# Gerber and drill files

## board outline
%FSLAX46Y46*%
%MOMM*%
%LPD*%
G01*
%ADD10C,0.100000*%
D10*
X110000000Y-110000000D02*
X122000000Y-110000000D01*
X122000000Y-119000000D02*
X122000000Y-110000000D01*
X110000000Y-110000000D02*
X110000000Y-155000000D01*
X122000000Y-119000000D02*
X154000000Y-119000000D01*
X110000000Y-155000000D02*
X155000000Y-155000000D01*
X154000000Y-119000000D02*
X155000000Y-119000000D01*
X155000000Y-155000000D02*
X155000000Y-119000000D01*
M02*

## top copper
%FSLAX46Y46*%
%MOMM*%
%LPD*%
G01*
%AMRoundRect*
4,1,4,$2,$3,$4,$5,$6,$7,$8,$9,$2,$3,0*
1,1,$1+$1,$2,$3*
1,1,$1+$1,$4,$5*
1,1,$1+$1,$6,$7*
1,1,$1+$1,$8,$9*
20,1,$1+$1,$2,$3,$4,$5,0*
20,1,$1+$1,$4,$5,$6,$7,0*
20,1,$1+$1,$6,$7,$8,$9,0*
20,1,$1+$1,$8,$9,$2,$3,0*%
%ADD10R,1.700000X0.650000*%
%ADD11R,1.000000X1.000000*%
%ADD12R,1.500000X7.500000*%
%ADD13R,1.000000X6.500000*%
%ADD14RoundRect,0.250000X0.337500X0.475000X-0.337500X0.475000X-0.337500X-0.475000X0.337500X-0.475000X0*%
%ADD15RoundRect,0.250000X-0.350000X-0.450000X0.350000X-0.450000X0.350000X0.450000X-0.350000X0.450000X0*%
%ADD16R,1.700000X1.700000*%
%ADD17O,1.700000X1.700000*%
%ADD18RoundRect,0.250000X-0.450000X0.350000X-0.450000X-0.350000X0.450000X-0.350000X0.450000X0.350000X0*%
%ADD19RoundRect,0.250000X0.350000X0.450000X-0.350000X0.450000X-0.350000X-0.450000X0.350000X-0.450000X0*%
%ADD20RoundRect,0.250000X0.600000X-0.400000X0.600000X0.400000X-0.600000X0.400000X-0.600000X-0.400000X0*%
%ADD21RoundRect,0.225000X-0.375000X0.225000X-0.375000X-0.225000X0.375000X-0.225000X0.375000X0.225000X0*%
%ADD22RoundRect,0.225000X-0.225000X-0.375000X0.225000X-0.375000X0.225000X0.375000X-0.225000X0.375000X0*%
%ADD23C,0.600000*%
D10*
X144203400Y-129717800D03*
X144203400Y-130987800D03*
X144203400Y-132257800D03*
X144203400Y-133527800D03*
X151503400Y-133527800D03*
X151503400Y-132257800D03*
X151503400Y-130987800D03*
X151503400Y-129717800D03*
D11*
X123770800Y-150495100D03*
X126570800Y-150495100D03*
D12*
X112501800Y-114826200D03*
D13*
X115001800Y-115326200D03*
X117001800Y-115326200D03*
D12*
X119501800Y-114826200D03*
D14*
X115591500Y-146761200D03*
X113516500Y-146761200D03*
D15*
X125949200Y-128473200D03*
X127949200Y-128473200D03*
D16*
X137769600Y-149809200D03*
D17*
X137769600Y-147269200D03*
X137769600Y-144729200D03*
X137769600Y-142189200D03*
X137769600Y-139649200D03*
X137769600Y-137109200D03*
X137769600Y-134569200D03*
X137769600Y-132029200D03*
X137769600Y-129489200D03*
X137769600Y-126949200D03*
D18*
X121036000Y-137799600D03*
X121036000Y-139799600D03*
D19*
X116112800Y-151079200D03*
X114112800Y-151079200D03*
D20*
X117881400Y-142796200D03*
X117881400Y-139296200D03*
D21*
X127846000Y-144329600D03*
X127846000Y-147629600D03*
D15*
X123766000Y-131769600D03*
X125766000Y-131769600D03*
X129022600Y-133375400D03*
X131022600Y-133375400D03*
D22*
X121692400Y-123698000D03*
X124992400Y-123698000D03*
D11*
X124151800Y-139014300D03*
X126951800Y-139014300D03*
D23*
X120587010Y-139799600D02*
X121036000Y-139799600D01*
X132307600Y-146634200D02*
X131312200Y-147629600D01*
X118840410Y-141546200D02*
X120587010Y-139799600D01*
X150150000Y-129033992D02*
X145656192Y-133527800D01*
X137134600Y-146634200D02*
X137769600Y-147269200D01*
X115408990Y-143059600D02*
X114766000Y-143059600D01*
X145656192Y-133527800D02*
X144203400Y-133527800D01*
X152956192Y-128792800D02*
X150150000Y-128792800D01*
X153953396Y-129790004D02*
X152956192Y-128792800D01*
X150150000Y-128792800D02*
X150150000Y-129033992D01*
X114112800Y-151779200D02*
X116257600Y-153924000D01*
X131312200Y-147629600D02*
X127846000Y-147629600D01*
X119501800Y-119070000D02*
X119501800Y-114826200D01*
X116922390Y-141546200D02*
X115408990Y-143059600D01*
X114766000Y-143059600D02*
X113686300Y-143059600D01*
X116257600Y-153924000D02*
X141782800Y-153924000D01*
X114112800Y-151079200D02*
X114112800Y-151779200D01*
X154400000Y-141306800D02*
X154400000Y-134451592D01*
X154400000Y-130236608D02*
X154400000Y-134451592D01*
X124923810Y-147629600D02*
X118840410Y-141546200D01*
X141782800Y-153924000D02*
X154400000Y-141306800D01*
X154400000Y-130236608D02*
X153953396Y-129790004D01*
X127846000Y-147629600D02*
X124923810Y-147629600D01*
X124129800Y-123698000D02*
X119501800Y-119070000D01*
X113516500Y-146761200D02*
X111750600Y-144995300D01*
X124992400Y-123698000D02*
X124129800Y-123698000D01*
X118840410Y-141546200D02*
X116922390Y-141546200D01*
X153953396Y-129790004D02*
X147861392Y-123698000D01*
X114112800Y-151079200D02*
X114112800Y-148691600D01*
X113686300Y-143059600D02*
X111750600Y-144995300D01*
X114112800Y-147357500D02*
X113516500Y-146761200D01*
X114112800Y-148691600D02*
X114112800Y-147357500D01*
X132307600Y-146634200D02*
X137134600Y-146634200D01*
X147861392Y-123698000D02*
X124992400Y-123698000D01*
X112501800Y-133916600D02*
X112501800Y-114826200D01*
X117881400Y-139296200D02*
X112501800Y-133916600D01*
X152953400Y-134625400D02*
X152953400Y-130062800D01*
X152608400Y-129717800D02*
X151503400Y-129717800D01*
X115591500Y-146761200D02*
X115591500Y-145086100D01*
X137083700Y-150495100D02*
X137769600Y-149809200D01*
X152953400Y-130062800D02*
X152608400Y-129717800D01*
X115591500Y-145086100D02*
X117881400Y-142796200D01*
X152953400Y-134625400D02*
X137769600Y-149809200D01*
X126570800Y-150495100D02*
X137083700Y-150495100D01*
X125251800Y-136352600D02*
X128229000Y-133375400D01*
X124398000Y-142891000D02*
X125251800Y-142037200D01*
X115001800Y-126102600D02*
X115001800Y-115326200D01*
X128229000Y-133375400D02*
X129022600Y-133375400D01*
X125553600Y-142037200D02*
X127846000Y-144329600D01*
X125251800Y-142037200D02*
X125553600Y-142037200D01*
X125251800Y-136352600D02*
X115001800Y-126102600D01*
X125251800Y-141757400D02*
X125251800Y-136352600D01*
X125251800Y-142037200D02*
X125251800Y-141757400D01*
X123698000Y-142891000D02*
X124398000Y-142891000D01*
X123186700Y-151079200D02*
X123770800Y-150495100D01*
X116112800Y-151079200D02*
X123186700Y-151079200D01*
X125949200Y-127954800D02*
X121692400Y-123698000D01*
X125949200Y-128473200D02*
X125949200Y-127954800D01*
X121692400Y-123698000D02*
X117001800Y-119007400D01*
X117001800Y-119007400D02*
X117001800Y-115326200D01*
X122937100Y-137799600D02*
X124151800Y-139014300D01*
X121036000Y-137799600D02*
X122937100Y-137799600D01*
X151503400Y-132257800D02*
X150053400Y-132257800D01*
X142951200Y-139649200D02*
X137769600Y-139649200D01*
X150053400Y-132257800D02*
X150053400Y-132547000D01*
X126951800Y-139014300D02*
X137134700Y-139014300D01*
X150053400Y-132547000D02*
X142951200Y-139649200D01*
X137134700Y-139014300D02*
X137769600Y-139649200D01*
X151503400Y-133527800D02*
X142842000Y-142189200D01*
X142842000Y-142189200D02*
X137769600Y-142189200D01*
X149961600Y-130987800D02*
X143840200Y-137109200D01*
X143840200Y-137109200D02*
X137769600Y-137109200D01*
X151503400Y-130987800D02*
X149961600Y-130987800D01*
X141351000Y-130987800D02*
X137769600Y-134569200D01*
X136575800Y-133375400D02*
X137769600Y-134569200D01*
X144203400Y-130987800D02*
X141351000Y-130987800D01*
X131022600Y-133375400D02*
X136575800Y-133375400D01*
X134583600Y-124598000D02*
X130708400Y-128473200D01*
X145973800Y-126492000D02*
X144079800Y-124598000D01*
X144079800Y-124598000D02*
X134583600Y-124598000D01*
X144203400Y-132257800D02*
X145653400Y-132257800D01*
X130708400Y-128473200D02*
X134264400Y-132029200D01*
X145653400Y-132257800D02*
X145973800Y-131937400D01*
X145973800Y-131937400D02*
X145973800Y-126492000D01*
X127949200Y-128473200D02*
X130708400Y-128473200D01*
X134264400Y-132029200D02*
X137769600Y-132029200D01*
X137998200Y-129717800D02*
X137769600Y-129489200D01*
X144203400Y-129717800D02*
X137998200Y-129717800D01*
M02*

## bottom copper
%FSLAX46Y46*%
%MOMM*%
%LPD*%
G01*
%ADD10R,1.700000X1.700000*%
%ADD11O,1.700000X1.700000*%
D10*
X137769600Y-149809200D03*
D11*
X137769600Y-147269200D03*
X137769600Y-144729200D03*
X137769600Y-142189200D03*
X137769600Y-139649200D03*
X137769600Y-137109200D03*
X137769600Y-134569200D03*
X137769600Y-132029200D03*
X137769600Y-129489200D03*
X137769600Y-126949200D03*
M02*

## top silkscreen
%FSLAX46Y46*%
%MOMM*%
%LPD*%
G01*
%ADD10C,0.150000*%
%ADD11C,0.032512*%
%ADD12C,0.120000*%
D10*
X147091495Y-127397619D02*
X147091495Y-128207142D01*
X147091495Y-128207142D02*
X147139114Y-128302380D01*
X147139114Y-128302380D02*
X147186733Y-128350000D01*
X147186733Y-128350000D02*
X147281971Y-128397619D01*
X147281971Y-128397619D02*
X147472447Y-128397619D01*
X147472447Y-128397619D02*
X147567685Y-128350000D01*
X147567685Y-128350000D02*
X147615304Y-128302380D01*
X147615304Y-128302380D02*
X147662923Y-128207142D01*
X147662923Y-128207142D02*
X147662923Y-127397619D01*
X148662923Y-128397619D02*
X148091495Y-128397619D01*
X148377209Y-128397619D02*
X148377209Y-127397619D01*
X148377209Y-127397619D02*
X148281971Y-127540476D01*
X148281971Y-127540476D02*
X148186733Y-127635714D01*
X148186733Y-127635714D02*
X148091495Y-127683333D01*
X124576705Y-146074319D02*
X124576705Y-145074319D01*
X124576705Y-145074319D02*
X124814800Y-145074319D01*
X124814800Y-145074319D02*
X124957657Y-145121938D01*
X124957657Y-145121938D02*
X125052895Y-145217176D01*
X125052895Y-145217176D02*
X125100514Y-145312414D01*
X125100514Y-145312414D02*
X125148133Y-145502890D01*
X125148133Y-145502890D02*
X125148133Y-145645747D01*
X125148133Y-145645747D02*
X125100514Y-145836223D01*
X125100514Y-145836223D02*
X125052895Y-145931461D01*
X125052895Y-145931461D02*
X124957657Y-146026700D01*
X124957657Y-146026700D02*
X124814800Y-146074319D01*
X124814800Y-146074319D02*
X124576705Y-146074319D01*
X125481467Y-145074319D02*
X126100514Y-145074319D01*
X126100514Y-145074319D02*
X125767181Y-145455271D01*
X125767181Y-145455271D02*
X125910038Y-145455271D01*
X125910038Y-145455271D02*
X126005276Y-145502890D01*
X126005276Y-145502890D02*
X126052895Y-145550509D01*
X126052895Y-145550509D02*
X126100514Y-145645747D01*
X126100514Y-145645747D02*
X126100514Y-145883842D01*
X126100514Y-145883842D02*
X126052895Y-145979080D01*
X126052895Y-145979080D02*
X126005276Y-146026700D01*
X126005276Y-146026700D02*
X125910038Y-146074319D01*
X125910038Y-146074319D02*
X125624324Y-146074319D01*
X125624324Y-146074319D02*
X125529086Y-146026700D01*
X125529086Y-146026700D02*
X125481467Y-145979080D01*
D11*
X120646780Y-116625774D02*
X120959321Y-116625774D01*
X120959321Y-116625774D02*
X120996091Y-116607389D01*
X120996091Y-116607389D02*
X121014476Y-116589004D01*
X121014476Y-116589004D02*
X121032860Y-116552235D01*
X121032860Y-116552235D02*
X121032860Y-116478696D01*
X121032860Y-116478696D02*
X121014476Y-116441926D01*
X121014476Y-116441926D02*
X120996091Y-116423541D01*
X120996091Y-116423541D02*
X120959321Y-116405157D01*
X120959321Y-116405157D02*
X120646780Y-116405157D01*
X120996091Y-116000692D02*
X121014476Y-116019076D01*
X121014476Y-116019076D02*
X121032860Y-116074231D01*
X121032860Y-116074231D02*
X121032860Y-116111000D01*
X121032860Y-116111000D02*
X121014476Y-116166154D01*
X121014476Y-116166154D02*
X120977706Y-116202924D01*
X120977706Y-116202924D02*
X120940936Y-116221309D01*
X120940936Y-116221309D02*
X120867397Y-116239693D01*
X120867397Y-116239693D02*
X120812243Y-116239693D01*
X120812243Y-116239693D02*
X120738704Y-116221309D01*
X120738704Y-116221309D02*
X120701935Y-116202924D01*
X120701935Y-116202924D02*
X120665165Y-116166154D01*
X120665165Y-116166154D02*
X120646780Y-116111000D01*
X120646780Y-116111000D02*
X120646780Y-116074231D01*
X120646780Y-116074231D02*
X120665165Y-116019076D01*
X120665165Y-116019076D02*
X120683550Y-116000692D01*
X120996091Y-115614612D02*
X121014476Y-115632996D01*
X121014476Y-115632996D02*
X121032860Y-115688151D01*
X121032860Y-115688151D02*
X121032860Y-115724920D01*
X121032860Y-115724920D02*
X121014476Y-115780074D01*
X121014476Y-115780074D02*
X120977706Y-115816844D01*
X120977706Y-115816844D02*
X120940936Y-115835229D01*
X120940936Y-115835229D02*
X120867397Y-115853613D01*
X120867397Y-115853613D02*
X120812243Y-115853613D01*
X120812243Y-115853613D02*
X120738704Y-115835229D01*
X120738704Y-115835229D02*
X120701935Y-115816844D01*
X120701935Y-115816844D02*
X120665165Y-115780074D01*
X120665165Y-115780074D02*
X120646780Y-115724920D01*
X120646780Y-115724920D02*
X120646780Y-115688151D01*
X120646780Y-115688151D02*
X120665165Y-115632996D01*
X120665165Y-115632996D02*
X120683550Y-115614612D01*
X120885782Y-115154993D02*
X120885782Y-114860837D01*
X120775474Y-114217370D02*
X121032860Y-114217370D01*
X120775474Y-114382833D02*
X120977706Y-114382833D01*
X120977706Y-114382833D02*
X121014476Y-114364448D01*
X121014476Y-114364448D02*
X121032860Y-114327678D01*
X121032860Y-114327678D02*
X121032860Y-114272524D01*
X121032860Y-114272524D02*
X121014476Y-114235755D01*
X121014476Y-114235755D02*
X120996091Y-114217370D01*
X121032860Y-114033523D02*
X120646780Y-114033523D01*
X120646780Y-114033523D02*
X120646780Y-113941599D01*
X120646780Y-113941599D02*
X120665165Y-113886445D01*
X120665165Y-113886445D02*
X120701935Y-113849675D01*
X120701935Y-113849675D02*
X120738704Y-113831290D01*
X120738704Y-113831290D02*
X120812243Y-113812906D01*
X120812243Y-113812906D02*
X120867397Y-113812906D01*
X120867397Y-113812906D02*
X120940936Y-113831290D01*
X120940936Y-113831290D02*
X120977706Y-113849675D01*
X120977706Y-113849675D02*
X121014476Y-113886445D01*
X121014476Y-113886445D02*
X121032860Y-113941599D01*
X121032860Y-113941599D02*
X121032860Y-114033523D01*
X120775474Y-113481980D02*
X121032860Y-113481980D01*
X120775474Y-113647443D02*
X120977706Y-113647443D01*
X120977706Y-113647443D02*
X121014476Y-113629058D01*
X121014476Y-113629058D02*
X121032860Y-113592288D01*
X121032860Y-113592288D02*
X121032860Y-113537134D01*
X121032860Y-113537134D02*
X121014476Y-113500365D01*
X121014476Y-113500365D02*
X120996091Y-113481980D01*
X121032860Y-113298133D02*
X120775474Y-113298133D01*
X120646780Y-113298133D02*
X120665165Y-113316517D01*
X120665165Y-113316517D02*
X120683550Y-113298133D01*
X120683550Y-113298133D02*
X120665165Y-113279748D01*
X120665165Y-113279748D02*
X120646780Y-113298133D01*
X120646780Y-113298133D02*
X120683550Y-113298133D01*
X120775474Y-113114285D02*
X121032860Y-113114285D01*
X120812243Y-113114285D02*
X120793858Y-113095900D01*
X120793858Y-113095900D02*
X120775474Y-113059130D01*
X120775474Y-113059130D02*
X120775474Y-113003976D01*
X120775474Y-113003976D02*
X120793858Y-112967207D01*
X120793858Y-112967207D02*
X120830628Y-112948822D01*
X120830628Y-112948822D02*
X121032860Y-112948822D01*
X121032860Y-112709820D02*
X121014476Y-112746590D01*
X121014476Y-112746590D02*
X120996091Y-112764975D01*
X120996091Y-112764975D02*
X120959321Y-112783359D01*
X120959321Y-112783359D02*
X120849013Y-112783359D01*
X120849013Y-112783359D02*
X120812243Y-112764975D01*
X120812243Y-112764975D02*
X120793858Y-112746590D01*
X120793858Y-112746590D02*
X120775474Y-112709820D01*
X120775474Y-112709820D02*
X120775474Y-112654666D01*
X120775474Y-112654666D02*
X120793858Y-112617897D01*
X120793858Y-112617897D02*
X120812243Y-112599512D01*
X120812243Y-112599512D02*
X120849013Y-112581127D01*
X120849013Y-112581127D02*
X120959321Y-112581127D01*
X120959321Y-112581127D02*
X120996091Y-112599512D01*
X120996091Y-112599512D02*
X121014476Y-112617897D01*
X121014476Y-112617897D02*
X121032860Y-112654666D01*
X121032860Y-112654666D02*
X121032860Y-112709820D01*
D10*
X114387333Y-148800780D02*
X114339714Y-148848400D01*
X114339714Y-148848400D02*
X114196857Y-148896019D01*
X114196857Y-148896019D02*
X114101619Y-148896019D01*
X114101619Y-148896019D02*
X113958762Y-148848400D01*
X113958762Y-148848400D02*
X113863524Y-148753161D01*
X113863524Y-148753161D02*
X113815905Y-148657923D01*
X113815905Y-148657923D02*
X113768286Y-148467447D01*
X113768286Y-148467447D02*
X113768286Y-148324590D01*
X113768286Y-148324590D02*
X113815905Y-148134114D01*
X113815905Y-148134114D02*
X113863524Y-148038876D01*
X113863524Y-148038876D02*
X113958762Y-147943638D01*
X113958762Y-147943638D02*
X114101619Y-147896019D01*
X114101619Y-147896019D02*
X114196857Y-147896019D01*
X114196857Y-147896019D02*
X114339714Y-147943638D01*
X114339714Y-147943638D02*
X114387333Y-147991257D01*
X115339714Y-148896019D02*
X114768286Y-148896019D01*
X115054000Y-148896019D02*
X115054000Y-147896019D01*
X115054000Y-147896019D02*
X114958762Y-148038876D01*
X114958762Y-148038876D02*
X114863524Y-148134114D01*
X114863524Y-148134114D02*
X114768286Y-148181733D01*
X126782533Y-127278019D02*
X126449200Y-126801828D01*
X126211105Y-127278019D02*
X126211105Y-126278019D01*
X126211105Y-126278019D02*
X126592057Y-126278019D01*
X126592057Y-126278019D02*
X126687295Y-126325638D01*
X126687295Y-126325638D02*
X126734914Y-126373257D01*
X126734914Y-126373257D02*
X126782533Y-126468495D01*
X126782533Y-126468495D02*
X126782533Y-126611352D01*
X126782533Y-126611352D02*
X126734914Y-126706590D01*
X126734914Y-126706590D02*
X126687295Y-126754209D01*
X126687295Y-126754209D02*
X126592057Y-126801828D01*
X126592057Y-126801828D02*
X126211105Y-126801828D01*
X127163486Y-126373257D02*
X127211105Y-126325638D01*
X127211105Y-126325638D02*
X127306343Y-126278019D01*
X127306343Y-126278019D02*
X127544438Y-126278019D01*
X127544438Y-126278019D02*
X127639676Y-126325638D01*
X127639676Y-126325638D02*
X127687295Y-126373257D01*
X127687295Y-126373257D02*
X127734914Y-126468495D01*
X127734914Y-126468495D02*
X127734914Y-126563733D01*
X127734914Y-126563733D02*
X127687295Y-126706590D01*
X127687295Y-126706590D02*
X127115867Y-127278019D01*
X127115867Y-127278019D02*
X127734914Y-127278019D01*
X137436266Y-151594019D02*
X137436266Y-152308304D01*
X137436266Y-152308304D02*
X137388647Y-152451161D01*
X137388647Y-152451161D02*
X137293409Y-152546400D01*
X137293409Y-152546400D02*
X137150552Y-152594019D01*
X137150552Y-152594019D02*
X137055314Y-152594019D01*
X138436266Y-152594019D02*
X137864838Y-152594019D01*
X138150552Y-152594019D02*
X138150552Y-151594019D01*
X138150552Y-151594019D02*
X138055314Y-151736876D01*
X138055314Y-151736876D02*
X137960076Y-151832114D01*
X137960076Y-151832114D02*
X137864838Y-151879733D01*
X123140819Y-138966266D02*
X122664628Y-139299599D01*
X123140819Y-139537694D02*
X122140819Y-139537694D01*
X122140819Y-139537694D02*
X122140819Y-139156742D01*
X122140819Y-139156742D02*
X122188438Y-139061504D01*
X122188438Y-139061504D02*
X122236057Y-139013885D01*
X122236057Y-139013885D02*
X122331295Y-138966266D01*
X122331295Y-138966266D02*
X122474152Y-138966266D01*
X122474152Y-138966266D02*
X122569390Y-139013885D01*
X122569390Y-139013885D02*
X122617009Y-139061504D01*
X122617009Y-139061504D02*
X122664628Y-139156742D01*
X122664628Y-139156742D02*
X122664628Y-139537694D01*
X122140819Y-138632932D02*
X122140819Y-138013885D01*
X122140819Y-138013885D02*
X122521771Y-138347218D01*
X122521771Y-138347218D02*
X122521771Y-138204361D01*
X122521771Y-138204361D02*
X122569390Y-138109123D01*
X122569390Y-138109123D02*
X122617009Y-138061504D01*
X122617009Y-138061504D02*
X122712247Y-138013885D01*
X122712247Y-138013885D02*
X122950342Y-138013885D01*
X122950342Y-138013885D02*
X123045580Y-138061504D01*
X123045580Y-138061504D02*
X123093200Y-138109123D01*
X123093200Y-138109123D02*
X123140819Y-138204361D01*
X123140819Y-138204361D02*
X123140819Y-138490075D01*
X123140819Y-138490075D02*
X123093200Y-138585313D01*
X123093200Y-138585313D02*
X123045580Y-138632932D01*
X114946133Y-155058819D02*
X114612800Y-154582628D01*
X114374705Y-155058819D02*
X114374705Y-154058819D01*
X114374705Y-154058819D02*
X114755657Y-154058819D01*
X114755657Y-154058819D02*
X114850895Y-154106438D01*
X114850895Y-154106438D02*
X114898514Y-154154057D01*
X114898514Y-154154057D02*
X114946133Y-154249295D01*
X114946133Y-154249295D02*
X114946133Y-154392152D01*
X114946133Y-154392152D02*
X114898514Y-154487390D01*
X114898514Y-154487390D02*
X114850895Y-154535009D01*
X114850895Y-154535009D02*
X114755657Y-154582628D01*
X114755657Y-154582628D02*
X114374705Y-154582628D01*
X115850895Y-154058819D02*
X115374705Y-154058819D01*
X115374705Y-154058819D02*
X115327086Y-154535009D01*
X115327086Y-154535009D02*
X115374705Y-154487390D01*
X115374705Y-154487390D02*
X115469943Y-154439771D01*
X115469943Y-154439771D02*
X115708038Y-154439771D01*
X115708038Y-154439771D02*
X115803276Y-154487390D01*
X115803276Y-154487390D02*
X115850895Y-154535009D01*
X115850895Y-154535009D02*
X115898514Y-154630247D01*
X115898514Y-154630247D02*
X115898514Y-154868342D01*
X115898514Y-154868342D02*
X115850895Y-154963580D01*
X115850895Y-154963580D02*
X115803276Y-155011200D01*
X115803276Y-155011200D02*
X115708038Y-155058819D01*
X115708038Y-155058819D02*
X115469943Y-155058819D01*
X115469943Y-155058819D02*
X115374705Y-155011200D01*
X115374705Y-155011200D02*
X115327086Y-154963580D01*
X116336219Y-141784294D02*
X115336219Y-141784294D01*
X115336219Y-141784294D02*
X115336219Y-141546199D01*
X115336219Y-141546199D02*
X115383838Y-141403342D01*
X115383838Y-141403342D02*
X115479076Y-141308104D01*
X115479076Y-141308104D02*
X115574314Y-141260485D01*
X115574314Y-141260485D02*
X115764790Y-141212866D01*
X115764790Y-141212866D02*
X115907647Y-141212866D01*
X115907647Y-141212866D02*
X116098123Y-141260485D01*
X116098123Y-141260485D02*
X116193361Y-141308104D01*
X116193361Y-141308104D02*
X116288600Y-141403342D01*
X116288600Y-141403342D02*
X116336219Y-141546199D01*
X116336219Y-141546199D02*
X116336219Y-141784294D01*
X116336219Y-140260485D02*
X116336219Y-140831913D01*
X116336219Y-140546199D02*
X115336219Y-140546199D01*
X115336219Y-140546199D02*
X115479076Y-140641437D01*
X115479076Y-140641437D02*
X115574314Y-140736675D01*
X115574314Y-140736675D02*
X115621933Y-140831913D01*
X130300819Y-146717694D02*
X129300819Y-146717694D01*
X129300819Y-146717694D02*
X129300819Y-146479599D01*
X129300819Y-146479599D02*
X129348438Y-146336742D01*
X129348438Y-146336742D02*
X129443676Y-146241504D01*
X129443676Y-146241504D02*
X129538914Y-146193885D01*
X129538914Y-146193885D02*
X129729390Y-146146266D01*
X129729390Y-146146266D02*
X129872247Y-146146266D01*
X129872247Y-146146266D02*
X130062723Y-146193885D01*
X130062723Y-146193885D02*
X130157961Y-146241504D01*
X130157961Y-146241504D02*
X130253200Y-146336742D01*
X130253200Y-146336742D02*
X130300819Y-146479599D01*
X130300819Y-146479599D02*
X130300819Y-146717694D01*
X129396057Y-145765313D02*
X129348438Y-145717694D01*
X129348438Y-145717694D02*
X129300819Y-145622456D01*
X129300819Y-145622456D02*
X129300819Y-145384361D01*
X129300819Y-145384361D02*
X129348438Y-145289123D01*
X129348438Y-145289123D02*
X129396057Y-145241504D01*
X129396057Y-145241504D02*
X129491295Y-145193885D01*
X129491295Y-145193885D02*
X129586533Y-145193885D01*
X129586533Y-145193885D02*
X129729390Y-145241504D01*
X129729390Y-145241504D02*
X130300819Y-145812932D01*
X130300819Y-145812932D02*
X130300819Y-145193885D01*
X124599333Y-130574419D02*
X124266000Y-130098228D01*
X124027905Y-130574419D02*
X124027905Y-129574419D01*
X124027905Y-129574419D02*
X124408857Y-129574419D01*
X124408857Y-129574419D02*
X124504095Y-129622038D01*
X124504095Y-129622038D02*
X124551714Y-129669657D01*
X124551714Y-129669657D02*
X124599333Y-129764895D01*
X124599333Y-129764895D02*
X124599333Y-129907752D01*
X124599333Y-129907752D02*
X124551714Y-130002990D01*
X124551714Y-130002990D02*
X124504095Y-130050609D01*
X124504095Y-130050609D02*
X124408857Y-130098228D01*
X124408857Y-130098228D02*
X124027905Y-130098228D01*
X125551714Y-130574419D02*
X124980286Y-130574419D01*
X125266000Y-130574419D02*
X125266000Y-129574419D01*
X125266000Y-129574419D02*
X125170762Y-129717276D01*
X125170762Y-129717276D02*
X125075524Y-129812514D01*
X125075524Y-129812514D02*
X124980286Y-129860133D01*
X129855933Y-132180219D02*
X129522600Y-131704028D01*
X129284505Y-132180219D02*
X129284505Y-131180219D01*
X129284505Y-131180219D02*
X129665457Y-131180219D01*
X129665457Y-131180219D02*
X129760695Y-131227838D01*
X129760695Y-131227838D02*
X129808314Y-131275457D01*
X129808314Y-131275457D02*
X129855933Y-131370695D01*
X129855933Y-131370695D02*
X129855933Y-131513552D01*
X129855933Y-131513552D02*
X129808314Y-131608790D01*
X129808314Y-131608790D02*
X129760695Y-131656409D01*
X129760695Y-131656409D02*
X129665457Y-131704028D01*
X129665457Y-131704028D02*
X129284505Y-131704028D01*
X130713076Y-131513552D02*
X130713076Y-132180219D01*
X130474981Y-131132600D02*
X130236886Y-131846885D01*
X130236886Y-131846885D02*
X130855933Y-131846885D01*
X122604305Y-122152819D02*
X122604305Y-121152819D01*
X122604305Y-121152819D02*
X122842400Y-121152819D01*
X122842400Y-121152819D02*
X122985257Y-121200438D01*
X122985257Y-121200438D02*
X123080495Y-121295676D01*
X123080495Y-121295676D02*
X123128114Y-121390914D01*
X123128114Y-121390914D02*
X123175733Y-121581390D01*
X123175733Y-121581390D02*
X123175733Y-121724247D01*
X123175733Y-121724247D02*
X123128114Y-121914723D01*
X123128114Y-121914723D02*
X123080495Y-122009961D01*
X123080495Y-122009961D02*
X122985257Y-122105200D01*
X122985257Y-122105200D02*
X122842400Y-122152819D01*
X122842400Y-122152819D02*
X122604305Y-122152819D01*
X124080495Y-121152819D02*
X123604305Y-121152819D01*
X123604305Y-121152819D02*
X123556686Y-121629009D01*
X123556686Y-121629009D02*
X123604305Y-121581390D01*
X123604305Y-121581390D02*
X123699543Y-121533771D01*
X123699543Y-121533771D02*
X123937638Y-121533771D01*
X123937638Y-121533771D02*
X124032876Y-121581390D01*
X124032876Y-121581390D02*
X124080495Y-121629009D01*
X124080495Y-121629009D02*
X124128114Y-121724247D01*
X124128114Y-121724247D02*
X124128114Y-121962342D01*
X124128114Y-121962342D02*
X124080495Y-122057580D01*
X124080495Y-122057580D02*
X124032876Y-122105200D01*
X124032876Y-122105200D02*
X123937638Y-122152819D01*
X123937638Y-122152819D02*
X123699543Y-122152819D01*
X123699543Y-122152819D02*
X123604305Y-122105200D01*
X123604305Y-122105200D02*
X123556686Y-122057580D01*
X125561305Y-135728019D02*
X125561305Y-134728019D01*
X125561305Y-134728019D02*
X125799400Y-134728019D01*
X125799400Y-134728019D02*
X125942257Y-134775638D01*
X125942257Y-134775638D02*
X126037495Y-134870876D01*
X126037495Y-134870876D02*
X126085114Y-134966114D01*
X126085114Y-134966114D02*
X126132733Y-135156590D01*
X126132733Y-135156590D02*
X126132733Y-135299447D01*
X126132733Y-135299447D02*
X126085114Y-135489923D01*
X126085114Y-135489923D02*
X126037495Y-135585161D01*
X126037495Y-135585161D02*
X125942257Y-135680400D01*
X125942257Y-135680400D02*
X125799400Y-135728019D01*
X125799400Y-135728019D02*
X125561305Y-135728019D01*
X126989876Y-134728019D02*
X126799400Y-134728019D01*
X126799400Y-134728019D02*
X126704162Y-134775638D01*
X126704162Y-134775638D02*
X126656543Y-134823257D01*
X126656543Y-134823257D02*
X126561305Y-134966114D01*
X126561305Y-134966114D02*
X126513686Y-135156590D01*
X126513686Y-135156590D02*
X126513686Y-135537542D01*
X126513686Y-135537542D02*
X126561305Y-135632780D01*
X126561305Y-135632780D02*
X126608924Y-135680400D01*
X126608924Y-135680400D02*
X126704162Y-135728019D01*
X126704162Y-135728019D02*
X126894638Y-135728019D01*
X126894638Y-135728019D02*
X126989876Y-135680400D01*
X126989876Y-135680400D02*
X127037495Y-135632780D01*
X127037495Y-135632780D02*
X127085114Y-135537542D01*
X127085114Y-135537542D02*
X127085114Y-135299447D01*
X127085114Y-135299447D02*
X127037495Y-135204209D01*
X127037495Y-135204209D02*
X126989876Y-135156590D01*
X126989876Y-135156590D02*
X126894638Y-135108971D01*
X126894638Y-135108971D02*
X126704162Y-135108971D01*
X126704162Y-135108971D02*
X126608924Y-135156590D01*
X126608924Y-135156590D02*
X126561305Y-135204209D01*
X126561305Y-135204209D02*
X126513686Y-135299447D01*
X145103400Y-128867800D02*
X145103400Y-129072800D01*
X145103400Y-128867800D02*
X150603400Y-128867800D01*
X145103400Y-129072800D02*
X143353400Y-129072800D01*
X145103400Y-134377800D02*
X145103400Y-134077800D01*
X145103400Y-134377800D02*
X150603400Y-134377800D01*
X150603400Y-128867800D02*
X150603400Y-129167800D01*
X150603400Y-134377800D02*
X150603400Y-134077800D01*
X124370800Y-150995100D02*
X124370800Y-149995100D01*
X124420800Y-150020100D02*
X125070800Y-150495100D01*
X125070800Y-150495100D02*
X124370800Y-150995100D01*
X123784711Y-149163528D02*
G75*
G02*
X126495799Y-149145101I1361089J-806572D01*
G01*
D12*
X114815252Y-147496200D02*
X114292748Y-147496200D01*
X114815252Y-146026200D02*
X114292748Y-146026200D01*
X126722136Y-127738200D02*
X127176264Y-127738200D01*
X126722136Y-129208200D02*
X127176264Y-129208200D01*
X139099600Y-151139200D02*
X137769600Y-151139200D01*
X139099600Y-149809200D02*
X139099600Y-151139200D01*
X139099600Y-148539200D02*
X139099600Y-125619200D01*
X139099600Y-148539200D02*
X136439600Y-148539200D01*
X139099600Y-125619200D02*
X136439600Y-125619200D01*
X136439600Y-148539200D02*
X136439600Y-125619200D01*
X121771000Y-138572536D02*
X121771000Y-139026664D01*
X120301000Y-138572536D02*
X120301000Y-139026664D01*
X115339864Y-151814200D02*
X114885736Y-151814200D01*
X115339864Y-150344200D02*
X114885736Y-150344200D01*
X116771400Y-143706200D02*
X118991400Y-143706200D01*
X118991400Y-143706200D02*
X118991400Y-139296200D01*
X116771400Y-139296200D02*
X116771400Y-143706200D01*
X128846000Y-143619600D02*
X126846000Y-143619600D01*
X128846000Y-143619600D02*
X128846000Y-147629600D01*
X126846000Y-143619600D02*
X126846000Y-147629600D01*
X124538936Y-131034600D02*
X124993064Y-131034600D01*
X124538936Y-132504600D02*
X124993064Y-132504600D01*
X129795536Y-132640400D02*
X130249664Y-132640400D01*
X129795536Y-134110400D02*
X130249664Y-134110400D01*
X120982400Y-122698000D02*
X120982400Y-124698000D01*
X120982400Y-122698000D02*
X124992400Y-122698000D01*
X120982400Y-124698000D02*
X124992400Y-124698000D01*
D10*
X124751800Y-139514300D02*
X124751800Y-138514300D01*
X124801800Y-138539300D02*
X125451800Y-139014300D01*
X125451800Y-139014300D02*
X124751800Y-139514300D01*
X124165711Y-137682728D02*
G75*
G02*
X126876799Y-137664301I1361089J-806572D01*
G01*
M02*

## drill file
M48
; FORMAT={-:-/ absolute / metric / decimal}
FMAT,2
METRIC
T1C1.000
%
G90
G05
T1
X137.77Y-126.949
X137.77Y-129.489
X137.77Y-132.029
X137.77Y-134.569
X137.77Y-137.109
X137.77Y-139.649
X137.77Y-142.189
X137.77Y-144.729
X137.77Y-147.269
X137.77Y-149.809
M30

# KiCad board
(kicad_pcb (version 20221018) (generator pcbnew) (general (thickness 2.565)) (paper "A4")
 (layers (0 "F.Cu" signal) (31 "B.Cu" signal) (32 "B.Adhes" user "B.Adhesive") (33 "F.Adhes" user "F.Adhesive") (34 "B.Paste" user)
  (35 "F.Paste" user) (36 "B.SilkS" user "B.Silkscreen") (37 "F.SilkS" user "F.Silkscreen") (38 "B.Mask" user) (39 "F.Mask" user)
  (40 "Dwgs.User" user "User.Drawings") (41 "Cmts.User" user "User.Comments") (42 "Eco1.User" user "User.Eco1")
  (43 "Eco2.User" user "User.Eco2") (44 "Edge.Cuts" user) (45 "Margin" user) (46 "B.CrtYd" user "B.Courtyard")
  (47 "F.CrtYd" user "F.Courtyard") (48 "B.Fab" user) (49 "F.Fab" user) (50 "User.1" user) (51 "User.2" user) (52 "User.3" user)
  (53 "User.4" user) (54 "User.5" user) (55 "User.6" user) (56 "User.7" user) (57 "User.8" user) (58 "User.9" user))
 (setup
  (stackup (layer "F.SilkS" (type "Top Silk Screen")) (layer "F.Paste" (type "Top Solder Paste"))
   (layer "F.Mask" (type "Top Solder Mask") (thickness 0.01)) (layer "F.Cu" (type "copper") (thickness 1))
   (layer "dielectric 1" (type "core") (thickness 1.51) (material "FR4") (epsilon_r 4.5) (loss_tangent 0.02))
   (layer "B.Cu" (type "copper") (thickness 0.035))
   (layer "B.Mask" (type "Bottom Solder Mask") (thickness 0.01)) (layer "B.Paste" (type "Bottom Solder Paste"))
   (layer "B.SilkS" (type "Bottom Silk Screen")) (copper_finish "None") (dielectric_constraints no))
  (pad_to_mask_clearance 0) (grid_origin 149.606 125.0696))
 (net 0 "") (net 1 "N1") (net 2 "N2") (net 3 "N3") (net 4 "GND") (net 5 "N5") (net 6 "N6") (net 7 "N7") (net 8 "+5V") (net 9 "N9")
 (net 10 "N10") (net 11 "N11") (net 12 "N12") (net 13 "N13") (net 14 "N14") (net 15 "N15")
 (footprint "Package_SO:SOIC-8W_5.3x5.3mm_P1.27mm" (layer "F.Cu") (at 147.8534 131.6228)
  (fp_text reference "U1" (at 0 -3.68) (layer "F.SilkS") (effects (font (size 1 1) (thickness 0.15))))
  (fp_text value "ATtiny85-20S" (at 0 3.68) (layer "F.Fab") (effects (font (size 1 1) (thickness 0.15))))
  (fp_line (start -2.75 -2.755) (end -2.75 -2.55) (stroke (width 0.15) (type solid)) (layer "F.SilkS"))
  (fp_line (start -2.75 -2.755) (end 2.75 -2.755) (stroke (width 0.15) (type solid)) (layer "F.SilkS"))
  (fp_line (start -2.75 -2.55) (end -4.5 -2.55) (stroke (width 0.15) (type solid)) (layer "F.SilkS"))
  (fp_line (start -2.75 2.755) (end -2.75 2.455) (stroke (width 0.15) (type solid)) (layer "F.SilkS"))
  (fp_line (start -2.75 2.755) (end 2.75 2.755) (stroke (width 0.15) (type solid)) (layer "F.SilkS"))
  (fp_line (start 2.75 -2.755) (end 2.75 -2.455) (stroke (width 0.15) (type solid)) (layer "F.SilkS"))
  (fp_line (start 2.75 2.755) (end 2.75 2.455) (stroke (width 0.15) (type solid)) (layer "F.SilkS"))
  (pad "1" smd rect (at -3.65 -1.905) (size 1.7 0.65) (layers "F.Cu" "F.Paste" "F.Mask") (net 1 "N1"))
  (pad "2" smd rect (at -3.65 -0.635) (size 1.7 0.65) (layers "F.Cu" "F.Paste" "F.Mask") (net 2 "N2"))
  (pad "3" smd rect (at -3.65 0.635) (size 1.7 0.65) (layers "F.Cu" "F.Paste" "F.Mask") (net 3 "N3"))
  (pad "4" smd rect (at -3.65 1.905) (size 1.7 0.65) (layers "F.Cu" "F.Paste" "F.Mask") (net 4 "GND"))
  (pad "5" smd rect (at 3.65 1.905) (size 1.7 0.65) (layers "F.Cu" "F.Paste" "F.Mask") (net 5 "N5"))
  (pad "6" smd rect (at 3.65 0.635) (size 1.7 0.65) (layers "F.Cu" "F.Paste" "F.Mask") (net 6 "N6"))
  (pad "7" smd rect (at 3.65 -0.635) (size 1.7 0.65) (layers "F.Cu" "F.Paste" "F.Mask") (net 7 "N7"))
  (pad "8" smd rect (at 3.65 -1.905) (size 1.7 0.65) (layers "F.Cu" "F.Paste" "F.Mask") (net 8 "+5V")))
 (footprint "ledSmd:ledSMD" (layer "F.Cu") (at 125.5708 150.4951)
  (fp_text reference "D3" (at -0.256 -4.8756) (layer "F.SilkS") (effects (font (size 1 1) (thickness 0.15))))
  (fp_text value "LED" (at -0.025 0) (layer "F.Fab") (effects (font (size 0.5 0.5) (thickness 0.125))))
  (fp_line (start -1.2 0.5) (end -1.2 -0.5) (stroke (width 0.15) (type solid)) (layer "F.SilkS"))
  (fp_line (start -1.15 -0.475) (end -0.5 0) (stroke (width 0.15) (type solid)) (layer "F.SilkS"))
  (fp_line (start -0.5 0) (end -1.2 0.5) (stroke (width 0.15) (type solid)) (layer "F.SilkS"))
  (fp_arc (start -1.786089 -1.331572) (mid -0.435753 -2.107089) (end 0.924999 -1.349999) (stroke (width 0.15) (type solid))
   (layer "F.SilkS"))
  (pad "1" smd rect (at -1.8 0) (size 1 1) (layers "F.Cu" "F.Paste" "F.Mask") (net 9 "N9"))
  (pad "2" smd rect (at 1 0) (size 1 1) (layers "F.Cu" "F.Paste" "F.Mask") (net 8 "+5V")))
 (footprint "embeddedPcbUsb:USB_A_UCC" (layer "F.Cu") (at 116.0018 115.0262 -90)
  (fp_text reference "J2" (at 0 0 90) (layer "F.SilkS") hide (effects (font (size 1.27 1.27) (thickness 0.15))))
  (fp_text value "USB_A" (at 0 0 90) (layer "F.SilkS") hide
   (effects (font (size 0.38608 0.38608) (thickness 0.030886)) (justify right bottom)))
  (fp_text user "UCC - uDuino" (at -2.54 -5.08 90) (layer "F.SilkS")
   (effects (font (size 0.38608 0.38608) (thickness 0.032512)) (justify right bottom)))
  (pad "1" smd rect (at -0.2 3.5 270) (size 7.5 1.5) (layers "F.Cu" "F.Paste" "F.Mask") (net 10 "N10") (solder_mask_margin 0.1016))
  (pad "2" smd rect (at 0.3 1 270) (size 6.5 1) (layers "F.Cu" "F.Paste" "F.Mask") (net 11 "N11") (solder_mask_margin 0.1016))
  (pad "3" smd rect (at 0.3 -1 270) (size 6.5 1) (layers "F.Cu" "F.Paste" "F.Mask") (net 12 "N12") (solder_mask_margin 0.1016))
  (pad "4" smd rect (at -0.2 -3.5 270) (size 7.5 1.5) (layers "F.Cu" "F.Paste" "F.Mask") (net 4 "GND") (solder_mask_margin 0.1016)))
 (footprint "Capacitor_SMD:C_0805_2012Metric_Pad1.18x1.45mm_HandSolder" (layer "F.Cu") (at 114.554 146.7612 180)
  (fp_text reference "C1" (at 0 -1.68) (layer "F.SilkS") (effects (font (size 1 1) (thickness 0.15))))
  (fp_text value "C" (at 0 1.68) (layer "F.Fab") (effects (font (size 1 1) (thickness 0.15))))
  (fp_line (start -0.261252 -0.735) (end 0.261252 -0.735) (stroke (width 0.12) (type solid)) (layer "F.SilkS"))
  (fp_line (start -0.261252 0.735) (end 0.261252 0.735) (stroke (width 0.12) (type solid)) (layer "F.SilkS"))
  (pad "1" smd roundrect (at -1.0375 0 180) (size 1.175 1.45) (layers "F.Cu" "F.Paste" "F.Mask") (roundrect_rratio 0.212766) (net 8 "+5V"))
  (pad "2" smd roundrect (at 1.0375 0 180) (size 1.175 1.45) (layers "F.Cu" "F.Paste" "F.Mask") (roundrect_rratio 0.212766) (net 4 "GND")))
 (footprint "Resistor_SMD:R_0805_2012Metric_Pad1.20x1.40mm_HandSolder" (layer "F.Cu") (at 126.9492 128.4732)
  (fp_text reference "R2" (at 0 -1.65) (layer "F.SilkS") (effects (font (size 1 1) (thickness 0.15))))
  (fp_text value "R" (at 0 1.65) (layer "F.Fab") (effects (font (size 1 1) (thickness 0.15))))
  (fp_line (start -0.227064 -0.735) (end 0.227064 -0.735) (stroke (width 0.12) (type solid)) (layer "F.SilkS"))
  (fp_line (start -0.227064 0.735) (end 0.227064 0.735) (stroke (width 0.12) (type solid)) (layer "F.SilkS"))
  (pad "1" smd roundrect (at -1 0) (size 1.2 1.4) (layers "F.Cu" "F.Paste" "F.Mask") (roundrect_rratio 0.208333) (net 12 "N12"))
  (pad "2" smd roundrect (at 1 0) (size 1.2 1.4) (layers "F.Cu" "F.Paste" "F.Mask") (roundrect_rratio 0.208333) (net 3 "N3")))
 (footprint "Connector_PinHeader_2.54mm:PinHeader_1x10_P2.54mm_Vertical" (layer "F.Cu") (at 137.7696 149.8092 180)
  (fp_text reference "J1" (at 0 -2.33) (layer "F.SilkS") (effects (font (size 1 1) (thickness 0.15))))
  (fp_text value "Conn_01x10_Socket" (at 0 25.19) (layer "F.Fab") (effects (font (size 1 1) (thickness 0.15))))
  (fp_line (start -1.33 -1.33) (end 0 -1.33) (stroke (width 0.12) (type solid)) (layer "F.SilkS"))
  (fp_line (start -1.33 0) (end -1.33 -1.33) (stroke (width 0.12) (type solid)) (layer "F.SilkS"))
  (fp_line (start -1.33 1.27) (end -1.33 24.19) (stroke (width 0.12) (type solid)) (layer "F.SilkS"))
  (fp_line (start -1.33 1.27) (end 1.33 1.27) (stroke (width 0.12) (type solid)) (layer "F.SilkS"))
  (fp_line (start -1.33 24.19) (end 1.33 24.19) (stroke (width 0.12) (type solid)) (layer "F.SilkS"))
  (fp_line (start 1.33 1.27) (end 1.33 24.19) (stroke (width 0.12) (type solid)) (layer "F.SilkS"))
  (pad "1" thru_hole rect (at 0 0 180) (size 1.7 1.7) (drill 1) (layers "*.Cu" "*.Mask") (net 8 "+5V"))
  (pad "2" thru_hole oval (at 0 2.54 180) (size 1.7 1.7) (drill 1) (layers "*.Cu" "*.Mask") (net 4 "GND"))
  (pad "3" thru_hole oval (at 0 5.08 180) (size 1.7 1.7) (drill 1) (layers "*.Cu" "*.Mask") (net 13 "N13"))
  (pad "4" thru_hole oval (at 0 7.62 180) (size 1.7 1.7) (drill 1) (layers "*.Cu" "*.Mask") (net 5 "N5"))
  (pad "5" thru_hole oval (at 0 10.16 180) (size 1.7 1.7) (drill 1) (layers "*.Cu" "*.Mask") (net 6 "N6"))
  (pad "6" thru_hole oval (at 0 12.7 180) (size 1.7 1.7) (drill 1) (layers "*.Cu" "*.Mask") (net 7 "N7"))
  (pad "7" thru_hole oval (at 0 15.24 180) (size 1.7 1.7) (drill 1) (layers "*.Cu" "*.Mask") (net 2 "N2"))
  (pad "8" thru_hole oval (at 0 17.78 180) (size 1.7 1.7) (drill 1) (layers "*.Cu" "*.Mask") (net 3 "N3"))
  (pad "9" thru_hole oval (at 0 20.32 180) (size 1.7 1.7) (drill 1) (layers "*.Cu" "*.Mask") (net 1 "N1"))
  (pad "10" thru_hole oval (at 0 22.86 180) (size 1.7 1.7) (drill 1) (layers "*.Cu" "*.Mask") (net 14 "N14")))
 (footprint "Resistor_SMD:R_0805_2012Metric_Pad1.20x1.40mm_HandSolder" (layer "F.Cu") (at 121.036 138.7996 -90)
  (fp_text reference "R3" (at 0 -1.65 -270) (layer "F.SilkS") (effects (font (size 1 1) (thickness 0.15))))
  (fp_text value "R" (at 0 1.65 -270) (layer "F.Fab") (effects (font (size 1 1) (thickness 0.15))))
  (fp_line (start -0.227064 -0.735) (end 0.227064 -0.735) (stroke (width 0.12) (type solid)) (layer "F.SilkS"))
  (fp_line (start -0.227064 0.735) (end 0.227064 0.735) (stroke (width 0.12) (type solid)) (layer "F.SilkS"))
  (pad "1" smd roundrect (at -1 0 270) (size 1.2 1.4) (layers "F.Cu" "F.Paste" "F.Mask") (roundrect_rratio 0.208333) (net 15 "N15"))
  (pad "2" smd roundrect (at 1 0 270) (size 1.2 1.4) (layers "F.Cu" "F.Paste" "F.Mask") (roundrect_rratio 0.208333) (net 4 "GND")))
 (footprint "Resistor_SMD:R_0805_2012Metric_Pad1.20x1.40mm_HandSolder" (layer "F.Cu") (at 115.1128 151.0792 180)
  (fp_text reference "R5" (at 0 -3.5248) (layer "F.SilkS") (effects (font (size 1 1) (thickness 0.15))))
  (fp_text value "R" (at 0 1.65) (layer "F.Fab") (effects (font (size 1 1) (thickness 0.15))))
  (fp_line (start -0.227064 -0.735) (end 0.227064 -0.735) (stroke (width 0.12) (type solid)) (layer "F.SilkS"))
  (fp_line (start -0.227064 0.735) (end 0.227064 0.735) (stroke (width 0.12) (type solid)) (layer "F.SilkS"))
  (pad "1" smd roundrect (at -1 0 180) (size 1.2 1.4) (layers "F.Cu" "F.Paste" "F.Mask") (roundrect_rratio 0.208333) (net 9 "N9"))
  (pad "2" smd roundrect (at 1 0 180) (size 1.2 1.4) (layers "F.Cu" "F.Paste" "F.Mask") (roundrect_rratio 0.208333) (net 4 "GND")))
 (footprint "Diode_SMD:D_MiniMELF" (layer "F.Cu") (at 117.8814 141.0462 90)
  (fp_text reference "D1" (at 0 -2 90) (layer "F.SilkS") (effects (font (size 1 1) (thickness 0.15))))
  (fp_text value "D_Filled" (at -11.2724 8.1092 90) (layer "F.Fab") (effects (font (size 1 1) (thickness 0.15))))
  (fp_line (start -2.66 -1.11) (end -2.66 1.11) (stroke (width 0.12) (type solid)) (layer "F.SilkS"))
  (fp_line (start -2.66 1.11) (end 1.75 1.11) (stroke (width 0.12) (type solid)) (layer "F.SilkS"))
  (fp_line (start 1.75 -1.11) (end -2.66 -1.11) (stroke (width 0.12) (type solid)) (layer "F.SilkS"))
  (pad "1" smd roundrect (at -1.75 0 90) (size 1.3 1.7) (layers "F.Cu" "F.Paste" "F.Mask") (roundrect_rratio 0.1923076923) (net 8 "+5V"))
  (pad "2" smd roundrect (at 1.75 0 90) (size 1.3 1.7) (layers "F.Cu" "F.Paste" "F.Mask") (roundrect_rratio 0.1923076923) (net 10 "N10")))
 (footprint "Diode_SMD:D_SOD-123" (layer "F.Cu") (at 127.846 145.9796 -90)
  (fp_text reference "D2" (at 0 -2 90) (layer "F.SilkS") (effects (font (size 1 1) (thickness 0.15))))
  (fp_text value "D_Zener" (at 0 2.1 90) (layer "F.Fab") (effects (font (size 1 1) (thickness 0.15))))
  (fp_line (start -2.36 -1) (end -2.36 1) (stroke (width 0.12) (type solid)) (layer "F.SilkS"))
  (fp_line (start -2.36 -1) (end 1.65 -1) (stroke (width 0.12) (type solid)) (layer "F.SilkS"))
  (fp_line (start -2.36 1) (end 1.65 1) (stroke (width 0.12) (type solid)) (layer "F.SilkS"))
  (pad "1" smd roundrect (at -1.65 0 270) (size 0.9 1.2) (layers "F.Cu" "F.Paste" "F.Mask") (roundrect_rratio 0.25) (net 11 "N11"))
  (pad "2" smd roundrect (at 1.65 0 270) (size 0.9 1.2) (layers "F.Cu" "F.Paste" "F.Mask") (roundrect_rratio 0.25) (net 4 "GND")))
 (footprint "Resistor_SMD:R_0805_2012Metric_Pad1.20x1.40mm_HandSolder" (layer "F.Cu") (at 124.766 131.7696)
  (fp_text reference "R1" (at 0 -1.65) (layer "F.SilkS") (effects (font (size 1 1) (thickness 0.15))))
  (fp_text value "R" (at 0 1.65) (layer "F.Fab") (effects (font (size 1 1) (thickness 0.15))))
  (fp_line (start -0.227064 -0.735) (end 0.227064 -0.735) (stroke (width 0.12) (type solid)) (layer "F.SilkS"))
  (fp_line (start -0.227064 0.735) (end 0.227064 0.735) (stroke (width 0.12) (type solid)) (layer "F.SilkS"))
  (pad "1" smd roundrect (at -1 0) (size 1.2 1.4) (layers "F.Cu" "F.Paste" "F.Mask") (roundrect_rratio 0.208333) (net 8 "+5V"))
  (pad "2" smd roundrect (at 1 0) (size 1.2 1.4) (layers "F.Cu" "F.Paste" "F.Mask") (roundrect_rratio 0.208333) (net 11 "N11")))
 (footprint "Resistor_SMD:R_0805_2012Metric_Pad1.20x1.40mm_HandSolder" (layer "F.Cu") (at 130.0226 133.3754)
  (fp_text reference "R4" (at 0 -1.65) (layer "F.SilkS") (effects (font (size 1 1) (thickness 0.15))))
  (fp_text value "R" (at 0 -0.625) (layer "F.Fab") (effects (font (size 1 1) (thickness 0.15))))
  (fp_line (start -0.227064 -0.735) (end 0.227064 -0.735) (stroke (width 0.12) (type solid)) (layer "F.SilkS"))
  (fp_line (start -0.227064 0.735) (end 0.227064 0.735) (stroke (width 0.12) (type solid)) (layer "F.SilkS"))
  (pad "1" smd roundrect (at -1 0) (size 1.2 1.4) (layers "F.Cu" "F.Paste" "F.Mask") (roundrect_rratio 0.208333) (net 11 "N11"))
  (pad "2" smd roundrect (at 1 0) (size 1.2 1.4) (layers "F.Cu" "F.Paste" "F.Mask") (roundrect_rratio 0.208333) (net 2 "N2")))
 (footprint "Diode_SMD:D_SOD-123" (layer "F.Cu") (at 123.3424 123.698)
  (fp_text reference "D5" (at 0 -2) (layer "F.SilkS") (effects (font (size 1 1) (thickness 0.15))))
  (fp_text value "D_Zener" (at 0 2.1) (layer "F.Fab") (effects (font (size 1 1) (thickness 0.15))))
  (fp_line (start -2.36 -1) (end -2.36 1) (stroke (width 0.12) (type solid)) (layer "F.SilkS"))
  (fp_line (start -2.36 -1) (end 1.65 -1) (stroke (width 0.12) (type solid)) (layer "F.SilkS"))
  (fp_line (start -2.36 1) (end 1.65 1) (stroke (width 0.12) (type solid)) (layer "F.SilkS"))
  (pad "1" smd roundrect (at -1.65 0) (size 0.9 1.2) (layers "F.Cu" "F.Paste" "F.Mask") (roundrect_rratio 0.25) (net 12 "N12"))
  (pad "2" smd roundrect (at 1.65 0) (size 0.9 1.2) (layers "F.Cu" "F.Paste" "F.Mask") (roundrect_rratio 0.25) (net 4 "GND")))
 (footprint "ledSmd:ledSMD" (layer "F.Cu") (at 125.9518 139.0143)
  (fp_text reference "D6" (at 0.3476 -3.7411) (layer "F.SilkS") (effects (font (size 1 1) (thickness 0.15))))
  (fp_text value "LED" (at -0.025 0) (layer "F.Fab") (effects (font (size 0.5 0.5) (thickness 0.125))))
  (fp_line (start -1.2 0.5) (end -1.2 -0.5) (stroke (width 0.15) (type solid)) (layer "F.SilkS"))
  (fp_line (start -1.15 -0.475) (end -0.5 0) (stroke (width 0.15) (type solid)) (layer "F.SilkS"))
  (fp_line (start -0.5 0) (end -1.2 0.5) (stroke (width 0.15) (type solid)) (layer "F.SilkS"))
  (fp_arc (start -1.786089 -1.331572) (mid -0.435753 -2.107089) (end 0.924999 -1.349999) (stroke (width 0.15) (type solid))
   (layer "F.SilkS"))
  (pad "1" smd rect (at -1.8 0) (size 1 1) (layers "F.Cu" "F.Paste" "F.Mask") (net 15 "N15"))
  (pad "2" smd rect (at 1 0) (size 1 1) (layers "F.Cu" "F.Paste" "F.Mask") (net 6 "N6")))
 (gr_line (start 110 110) (end 122 110) (stroke (width 0.1) (type default)) (layer "Edge.Cuts"))
 (gr_line (start 122 119) (end 122 110) (stroke (width 0.1) (type default)) (layer "Edge.Cuts"))
 (gr_line (start 110 110) (end 110 155) (stroke (width 0.1) (type default)) (layer "Edge.Cuts"))
 (gr_line (start 122 119) (end 154 119) (stroke (width 0.1) (type default)) (layer "Edge.Cuts"))
 (gr_line (start 110 155) (end 155 155) (stroke (width 0.1) (type default)) (layer "Edge.Cuts"))
 (gr_line (start 154 119) (end 155 119) (stroke (width 0.1) (type default)) (layer "Edge.Cuts"))
 (gr_line (start 155 155) (end 155 119) (stroke (width 0.1) (type default)) (layer "Edge.Cuts"))
 (segment (start 120.58701 139.7996) (end 121.036 139.7996) (width 0.6) (layer "F.Cu") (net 4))
 (segment (start 132.3076 146.6342) (end 131.3122 147.6296) (width 0.6) (layer "F.Cu") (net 4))
 (segment (start 118.84041 141.5462) (end 120.58701 139.7996) (width 0.6) (layer "F.Cu") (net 4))
 (segment (start 150.15 129.033992) (end 145.656192 133.5278) (width 0.6) (layer "F.Cu") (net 4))
 (segment (start 137.1346 146.6342) (end 137.7696 147.2692) (width 0.6) (layer "F.Cu") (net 4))
 (segment (start 115.40899 143.0596) (end 114.766 143.0596) (width 0.6) (layer "F.Cu") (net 4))
 (segment (start 145.656192 133.5278) (end 144.2034 133.5278) (width 0.6) (layer "F.Cu") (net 4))
 (segment (start 152.956192 128.7928) (end 150.15 128.7928) (width 0.6) (layer "F.Cu") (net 4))
 (segment (start 153.953396 129.790004) (end 152.956192 128.7928) (width 0.6) (layer "F.Cu") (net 4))
 (segment (start 150.15 128.7928) (end 150.15 129.033992) (width 0.6) (layer "F.Cu") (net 4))
 (segment (start 114.1128 151.7792) (end 116.2576 153.924) (width 0.6) (layer "F.Cu") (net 4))
 (segment (start 131.3122 147.6296) (end 127.846 147.6296) (width 0.6) (layer "F.Cu") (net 4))
 (segment (start 119.5018 119.07) (end 119.5018 114.8262) (width 0.6) (layer "F.Cu") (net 4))
 (segment (start 116.92239 141.5462) (end 115.40899 143.0596) (width 0.6) (layer "F.Cu") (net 4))
 (segment (start 114.766 143.0596) (end 113.6863 143.0596) (width 0.6) (layer "F.Cu") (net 4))
 (segment (start 116.2576 153.924) (end 141.7828 153.924) (width 0.6) (layer "F.Cu") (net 4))
 (segment (start 114.1128 151.0792) (end 114.1128 151.7792) (width 0.6) (layer "F.Cu") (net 4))
 (segment (start 154.4 141.3068) (end 154.4 134.451592) (width 0.6) (layer "F.Cu") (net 4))
 (segment (start 154.4 130.236608) (end 154.4 134.451592) (width 0.6) (layer "F.Cu") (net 4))
 (segment (start 124.92381 147.6296) (end 118.84041 141.5462) (width 0.6) (layer "F.Cu") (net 4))
 (segment (start 141.7828 153.924) (end 154.4 141.3068) (width 0.6) (layer "F.Cu") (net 4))
 (segment (start 154.4 130.236608) (end 153.953396 129.790004) (width 0.6) (layer "F.Cu") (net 4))
 (segment (start 127.846 147.6296) (end 124.92381 147.6296) (width 0.6) (layer "F.Cu") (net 4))
 (segment (start 124.1298 123.698) (end 119.5018 119.07) (width 0.6) (layer "F.Cu") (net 4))
 (segment (start 113.5165 146.7612) (end 111.7506 144.9953) (width 0.6) (layer "F.Cu") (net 4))
 (segment (start 124.9924 123.698) (end 124.1298 123.698) (width 0.6) (layer "F.Cu") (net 4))
 (segment (start 118.84041 141.5462) (end 116.92239 141.5462) (width 0.6) (layer "F.Cu") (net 4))
 (segment (start 153.953396 129.790004) (end 147.861392 123.698) (width 0.6) (layer "F.Cu") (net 4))
 (segment (start 114.1128 151.0792) (end 114.1128 148.6916) (width 0.6) (layer "F.Cu") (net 4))
 (segment (start 113.6863 143.0596) (end 111.7506 144.9953) (width 0.6) (layer "F.Cu") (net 4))
 (segment (start 114.1128 147.3575) (end 113.5165 146.7612) (width 0.6) (layer "F.Cu") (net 4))
 (segment (start 114.1128 148.6916) (end 114.1128 147.3575) (width 0.6) (layer "F.Cu") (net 4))
 (segment (start 132.3076 146.6342) (end 137.1346 146.6342) (width 0.6) (layer "F.Cu") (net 4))
 (segment (start 147.861392 123.698) (end 124.9924 123.698) (width 0.6) (layer "F.Cu") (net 4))
 (segment (start 112.5018 133.9166) (end 112.5018 114.8262) (width 0.6) (layer "F.Cu") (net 10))
 (segment (start 117.8814 139.2962) (end 112.5018 133.9166) (width 0.6) (layer "F.Cu") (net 10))
 (segment (start 152.9534 134.6254) (end 152.9534 130.0628) (width 0.6) (layer "F.Cu") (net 8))
 (segment (start 152.6084 129.7178) (end 151.5034 129.7178) (width 0.6) (layer "F.Cu") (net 8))
 (segment (start 115.5915 146.7612) (end 115.5915 145.0861) (width 0.6) (layer "F.Cu") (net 8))
 (segment (start 137.0837 150.4951) (end 137.7696 149.8092) (width 0.6) (layer "F.Cu") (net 8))
 (segment (start 152.9534 130.0628) (end 152.6084 129.7178) (width 0.6) (layer "F.Cu") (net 8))
 (segment (start 115.5915 145.0861) (end 117.8814 142.7962) (width 0.6) (layer "F.Cu") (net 8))
 (segment (start 152.9534 134.6254) (end 137.7696 149.8092) (width 0.6) (layer "F.Cu") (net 8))
 (segment (start 126.5708 150.4951) (end 137.0837 150.4951) (width 0.6) (layer "F.Cu") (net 8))
 (segment (start 125.2518 136.3526) (end 128.229 133.3754) (width 0.6) (layer "F.Cu") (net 11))
 (segment (start 124.398 142.891) (end 125.2518 142.0372) (width 0.6) (layer "F.Cu") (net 11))
 (segment (start 115.0018 126.1026) (end 115.0018 115.3262) (width 0.6) (layer "F.Cu") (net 11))
 (segment (start 128.229 133.3754) (end 129.0226 133.3754) (width 0.6) (layer "F.Cu") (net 11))
 (segment (start 125.5536 142.0372) (end 127.846 144.3296) (width 0.6) (layer "F.Cu") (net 11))
 (segment (start 125.2518 142.0372) (end 125.5536 142.0372) (width 0.6) (layer "F.Cu") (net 11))
 (segment (start 125.2518 136.3526) (end 115.0018 126.1026) (width 0.6) (layer "F.Cu") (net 11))
 (segment (start 125.2518 141.7574) (end 125.2518 136.3526) (width 0.6) (layer "F.Cu") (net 11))
 (segment (start 125.2518 142.0372) (end 125.2518 141.7574) (width 0.6) (layer "F.Cu") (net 11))
 (segment (start 123.698 142.891) (end 124.398 142.891) (width 0.6) (layer "F.Cu") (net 11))
 (segment (start 123.1867 151.0792) (end 123.7708 150.4951) (width 0.6) (layer "F.Cu") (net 9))
 (segment (start 116.1128 151.0792) (end 123.1867 151.0792) (width 0.6) (layer "F.Cu") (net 9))
 (segment (start 125.9492 127.9548) (end 121.6924 123.698) (width 0.6) (layer "F.Cu") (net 12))
 (segment (start 125.9492 128.4732) (end 125.9492 127.9548) (width 0.6) (layer "F.Cu") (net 12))
 (segment (start 121.6924 123.698) (end 117.0018 119.0074) (width 0.6) (layer "F.Cu") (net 12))
 (segment (start 117.0018 119.0074) (end 117.0018 115.3262) (width 0.6) (layer "F.Cu") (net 12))
 (segment (start 122.9371 137.7996) (end 124.1518 139.0143) (width 0.6) (layer "F.Cu") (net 15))
 (segment (start 121.036 137.7996) (end 122.9371 137.7996) (width 0.6) (layer "F.Cu") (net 15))
 (segment (start 151.5034 132.2578) (end 150.0534 132.2578) (width 0.6) (layer "F.Cu") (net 6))
 (segment (start 142.9512 139.6492) (end 137.7696 139.6492) (width 0.6) (layer "F.Cu") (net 6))
 (segment (start 150.0534 132.2578) (end 150.0534 132.547) (width 0.6) (layer "F.Cu") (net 6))
 (segment (start 126.9518 139.0143) (end 137.1347 139.0143) (width 0.6) (layer "F.Cu") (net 6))
 (segment (start 150.0534 132.547) (end 142.9512 139.6492) (width 0.6) (layer "F.Cu") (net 6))
 (segment (start 137.1347 139.0143) (end 137.7696 139.6492) (width 0.6) (layer "F.Cu") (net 6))
 (segment (start 151.5034 133.5278) (end 142.842 142.1892) (width 0.6) (layer "F.Cu") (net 5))
 (segment (start 142.842 142.1892) (end 137.7696 142.1892) (width 0.6) (layer "F.Cu") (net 5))
 (segment (start 149.9616 130.9878) (end 143.8402 137.1092) (width 0.6) (layer "F.Cu") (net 7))
 (segment (start 143.8402 137.1092) (end 137.7696 137.1092) (width 0.6) (layer "F.Cu") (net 7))
 (segment (start 151.5034 130.9878) (end 149.9616 130.9878) (width 0.6) (layer "F.Cu") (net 7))
 (segment (start 141.351 130.9878) (end 137.7696 134.5692) (width 0.6) (layer "F.Cu") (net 2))
 (segment (start 136.5758 133.3754) (end 137.7696 134.5692) (width 0.6) (layer "F.Cu") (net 2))
 (segment (start 144.2034 130.9878) (end 141.351 130.9878) (width 0.6) (layer "F.Cu") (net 2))
 (segment (start 131.0226 133.3754) (end 136.5758 133.3754) (width 0.6) (layer "F.Cu") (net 2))
 (segment (start 134.5836 124.598) (end 130.7084 128.4732) (width 0.6) (layer "F.Cu") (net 3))
 (segment (start 145.9738 126.492) (end 144.0798 124.598) (width 0.6) (layer "F.Cu") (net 3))
 (segment (start 144.0798 124.598) (end 134.5836 124.598) (width 0.6) (layer "F.Cu") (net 3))
 (segment (start 144.2034 132.2578) (end 145.6534 132.2578) (width 0.6) (layer "F.Cu") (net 3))
 (segment (start 130.7084 128.4732) (end 134.2644 132.0292) (width 0.6) (layer "F.Cu") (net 3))
 (segment (start 145.6534 132.2578) (end 145.9738 131.9374) (width 0.6) (layer "F.Cu") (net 3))
 (segment (start 145.9738 131.9374) (end 145.9738 126.492) (width 0.6) (layer "F.Cu") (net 3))
 (segment (start 127.9492 128.4732) (end 130.7084 128.4732) (width 0.6) (layer "F.Cu") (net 3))
 (segment (start 134.2644 132.0292) (end 137.7696 132.0292) (width 0.6) (layer "F.Cu") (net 3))
 (segment (start 137.9982 129.7178) (end 137.7696 129.4892) (width 0.6) (layer "F.Cu") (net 1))
 (segment (start 144.2034 129.7178) (end 137.9982 129.7178) (width 0.6) (layer "F.Cu") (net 1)))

